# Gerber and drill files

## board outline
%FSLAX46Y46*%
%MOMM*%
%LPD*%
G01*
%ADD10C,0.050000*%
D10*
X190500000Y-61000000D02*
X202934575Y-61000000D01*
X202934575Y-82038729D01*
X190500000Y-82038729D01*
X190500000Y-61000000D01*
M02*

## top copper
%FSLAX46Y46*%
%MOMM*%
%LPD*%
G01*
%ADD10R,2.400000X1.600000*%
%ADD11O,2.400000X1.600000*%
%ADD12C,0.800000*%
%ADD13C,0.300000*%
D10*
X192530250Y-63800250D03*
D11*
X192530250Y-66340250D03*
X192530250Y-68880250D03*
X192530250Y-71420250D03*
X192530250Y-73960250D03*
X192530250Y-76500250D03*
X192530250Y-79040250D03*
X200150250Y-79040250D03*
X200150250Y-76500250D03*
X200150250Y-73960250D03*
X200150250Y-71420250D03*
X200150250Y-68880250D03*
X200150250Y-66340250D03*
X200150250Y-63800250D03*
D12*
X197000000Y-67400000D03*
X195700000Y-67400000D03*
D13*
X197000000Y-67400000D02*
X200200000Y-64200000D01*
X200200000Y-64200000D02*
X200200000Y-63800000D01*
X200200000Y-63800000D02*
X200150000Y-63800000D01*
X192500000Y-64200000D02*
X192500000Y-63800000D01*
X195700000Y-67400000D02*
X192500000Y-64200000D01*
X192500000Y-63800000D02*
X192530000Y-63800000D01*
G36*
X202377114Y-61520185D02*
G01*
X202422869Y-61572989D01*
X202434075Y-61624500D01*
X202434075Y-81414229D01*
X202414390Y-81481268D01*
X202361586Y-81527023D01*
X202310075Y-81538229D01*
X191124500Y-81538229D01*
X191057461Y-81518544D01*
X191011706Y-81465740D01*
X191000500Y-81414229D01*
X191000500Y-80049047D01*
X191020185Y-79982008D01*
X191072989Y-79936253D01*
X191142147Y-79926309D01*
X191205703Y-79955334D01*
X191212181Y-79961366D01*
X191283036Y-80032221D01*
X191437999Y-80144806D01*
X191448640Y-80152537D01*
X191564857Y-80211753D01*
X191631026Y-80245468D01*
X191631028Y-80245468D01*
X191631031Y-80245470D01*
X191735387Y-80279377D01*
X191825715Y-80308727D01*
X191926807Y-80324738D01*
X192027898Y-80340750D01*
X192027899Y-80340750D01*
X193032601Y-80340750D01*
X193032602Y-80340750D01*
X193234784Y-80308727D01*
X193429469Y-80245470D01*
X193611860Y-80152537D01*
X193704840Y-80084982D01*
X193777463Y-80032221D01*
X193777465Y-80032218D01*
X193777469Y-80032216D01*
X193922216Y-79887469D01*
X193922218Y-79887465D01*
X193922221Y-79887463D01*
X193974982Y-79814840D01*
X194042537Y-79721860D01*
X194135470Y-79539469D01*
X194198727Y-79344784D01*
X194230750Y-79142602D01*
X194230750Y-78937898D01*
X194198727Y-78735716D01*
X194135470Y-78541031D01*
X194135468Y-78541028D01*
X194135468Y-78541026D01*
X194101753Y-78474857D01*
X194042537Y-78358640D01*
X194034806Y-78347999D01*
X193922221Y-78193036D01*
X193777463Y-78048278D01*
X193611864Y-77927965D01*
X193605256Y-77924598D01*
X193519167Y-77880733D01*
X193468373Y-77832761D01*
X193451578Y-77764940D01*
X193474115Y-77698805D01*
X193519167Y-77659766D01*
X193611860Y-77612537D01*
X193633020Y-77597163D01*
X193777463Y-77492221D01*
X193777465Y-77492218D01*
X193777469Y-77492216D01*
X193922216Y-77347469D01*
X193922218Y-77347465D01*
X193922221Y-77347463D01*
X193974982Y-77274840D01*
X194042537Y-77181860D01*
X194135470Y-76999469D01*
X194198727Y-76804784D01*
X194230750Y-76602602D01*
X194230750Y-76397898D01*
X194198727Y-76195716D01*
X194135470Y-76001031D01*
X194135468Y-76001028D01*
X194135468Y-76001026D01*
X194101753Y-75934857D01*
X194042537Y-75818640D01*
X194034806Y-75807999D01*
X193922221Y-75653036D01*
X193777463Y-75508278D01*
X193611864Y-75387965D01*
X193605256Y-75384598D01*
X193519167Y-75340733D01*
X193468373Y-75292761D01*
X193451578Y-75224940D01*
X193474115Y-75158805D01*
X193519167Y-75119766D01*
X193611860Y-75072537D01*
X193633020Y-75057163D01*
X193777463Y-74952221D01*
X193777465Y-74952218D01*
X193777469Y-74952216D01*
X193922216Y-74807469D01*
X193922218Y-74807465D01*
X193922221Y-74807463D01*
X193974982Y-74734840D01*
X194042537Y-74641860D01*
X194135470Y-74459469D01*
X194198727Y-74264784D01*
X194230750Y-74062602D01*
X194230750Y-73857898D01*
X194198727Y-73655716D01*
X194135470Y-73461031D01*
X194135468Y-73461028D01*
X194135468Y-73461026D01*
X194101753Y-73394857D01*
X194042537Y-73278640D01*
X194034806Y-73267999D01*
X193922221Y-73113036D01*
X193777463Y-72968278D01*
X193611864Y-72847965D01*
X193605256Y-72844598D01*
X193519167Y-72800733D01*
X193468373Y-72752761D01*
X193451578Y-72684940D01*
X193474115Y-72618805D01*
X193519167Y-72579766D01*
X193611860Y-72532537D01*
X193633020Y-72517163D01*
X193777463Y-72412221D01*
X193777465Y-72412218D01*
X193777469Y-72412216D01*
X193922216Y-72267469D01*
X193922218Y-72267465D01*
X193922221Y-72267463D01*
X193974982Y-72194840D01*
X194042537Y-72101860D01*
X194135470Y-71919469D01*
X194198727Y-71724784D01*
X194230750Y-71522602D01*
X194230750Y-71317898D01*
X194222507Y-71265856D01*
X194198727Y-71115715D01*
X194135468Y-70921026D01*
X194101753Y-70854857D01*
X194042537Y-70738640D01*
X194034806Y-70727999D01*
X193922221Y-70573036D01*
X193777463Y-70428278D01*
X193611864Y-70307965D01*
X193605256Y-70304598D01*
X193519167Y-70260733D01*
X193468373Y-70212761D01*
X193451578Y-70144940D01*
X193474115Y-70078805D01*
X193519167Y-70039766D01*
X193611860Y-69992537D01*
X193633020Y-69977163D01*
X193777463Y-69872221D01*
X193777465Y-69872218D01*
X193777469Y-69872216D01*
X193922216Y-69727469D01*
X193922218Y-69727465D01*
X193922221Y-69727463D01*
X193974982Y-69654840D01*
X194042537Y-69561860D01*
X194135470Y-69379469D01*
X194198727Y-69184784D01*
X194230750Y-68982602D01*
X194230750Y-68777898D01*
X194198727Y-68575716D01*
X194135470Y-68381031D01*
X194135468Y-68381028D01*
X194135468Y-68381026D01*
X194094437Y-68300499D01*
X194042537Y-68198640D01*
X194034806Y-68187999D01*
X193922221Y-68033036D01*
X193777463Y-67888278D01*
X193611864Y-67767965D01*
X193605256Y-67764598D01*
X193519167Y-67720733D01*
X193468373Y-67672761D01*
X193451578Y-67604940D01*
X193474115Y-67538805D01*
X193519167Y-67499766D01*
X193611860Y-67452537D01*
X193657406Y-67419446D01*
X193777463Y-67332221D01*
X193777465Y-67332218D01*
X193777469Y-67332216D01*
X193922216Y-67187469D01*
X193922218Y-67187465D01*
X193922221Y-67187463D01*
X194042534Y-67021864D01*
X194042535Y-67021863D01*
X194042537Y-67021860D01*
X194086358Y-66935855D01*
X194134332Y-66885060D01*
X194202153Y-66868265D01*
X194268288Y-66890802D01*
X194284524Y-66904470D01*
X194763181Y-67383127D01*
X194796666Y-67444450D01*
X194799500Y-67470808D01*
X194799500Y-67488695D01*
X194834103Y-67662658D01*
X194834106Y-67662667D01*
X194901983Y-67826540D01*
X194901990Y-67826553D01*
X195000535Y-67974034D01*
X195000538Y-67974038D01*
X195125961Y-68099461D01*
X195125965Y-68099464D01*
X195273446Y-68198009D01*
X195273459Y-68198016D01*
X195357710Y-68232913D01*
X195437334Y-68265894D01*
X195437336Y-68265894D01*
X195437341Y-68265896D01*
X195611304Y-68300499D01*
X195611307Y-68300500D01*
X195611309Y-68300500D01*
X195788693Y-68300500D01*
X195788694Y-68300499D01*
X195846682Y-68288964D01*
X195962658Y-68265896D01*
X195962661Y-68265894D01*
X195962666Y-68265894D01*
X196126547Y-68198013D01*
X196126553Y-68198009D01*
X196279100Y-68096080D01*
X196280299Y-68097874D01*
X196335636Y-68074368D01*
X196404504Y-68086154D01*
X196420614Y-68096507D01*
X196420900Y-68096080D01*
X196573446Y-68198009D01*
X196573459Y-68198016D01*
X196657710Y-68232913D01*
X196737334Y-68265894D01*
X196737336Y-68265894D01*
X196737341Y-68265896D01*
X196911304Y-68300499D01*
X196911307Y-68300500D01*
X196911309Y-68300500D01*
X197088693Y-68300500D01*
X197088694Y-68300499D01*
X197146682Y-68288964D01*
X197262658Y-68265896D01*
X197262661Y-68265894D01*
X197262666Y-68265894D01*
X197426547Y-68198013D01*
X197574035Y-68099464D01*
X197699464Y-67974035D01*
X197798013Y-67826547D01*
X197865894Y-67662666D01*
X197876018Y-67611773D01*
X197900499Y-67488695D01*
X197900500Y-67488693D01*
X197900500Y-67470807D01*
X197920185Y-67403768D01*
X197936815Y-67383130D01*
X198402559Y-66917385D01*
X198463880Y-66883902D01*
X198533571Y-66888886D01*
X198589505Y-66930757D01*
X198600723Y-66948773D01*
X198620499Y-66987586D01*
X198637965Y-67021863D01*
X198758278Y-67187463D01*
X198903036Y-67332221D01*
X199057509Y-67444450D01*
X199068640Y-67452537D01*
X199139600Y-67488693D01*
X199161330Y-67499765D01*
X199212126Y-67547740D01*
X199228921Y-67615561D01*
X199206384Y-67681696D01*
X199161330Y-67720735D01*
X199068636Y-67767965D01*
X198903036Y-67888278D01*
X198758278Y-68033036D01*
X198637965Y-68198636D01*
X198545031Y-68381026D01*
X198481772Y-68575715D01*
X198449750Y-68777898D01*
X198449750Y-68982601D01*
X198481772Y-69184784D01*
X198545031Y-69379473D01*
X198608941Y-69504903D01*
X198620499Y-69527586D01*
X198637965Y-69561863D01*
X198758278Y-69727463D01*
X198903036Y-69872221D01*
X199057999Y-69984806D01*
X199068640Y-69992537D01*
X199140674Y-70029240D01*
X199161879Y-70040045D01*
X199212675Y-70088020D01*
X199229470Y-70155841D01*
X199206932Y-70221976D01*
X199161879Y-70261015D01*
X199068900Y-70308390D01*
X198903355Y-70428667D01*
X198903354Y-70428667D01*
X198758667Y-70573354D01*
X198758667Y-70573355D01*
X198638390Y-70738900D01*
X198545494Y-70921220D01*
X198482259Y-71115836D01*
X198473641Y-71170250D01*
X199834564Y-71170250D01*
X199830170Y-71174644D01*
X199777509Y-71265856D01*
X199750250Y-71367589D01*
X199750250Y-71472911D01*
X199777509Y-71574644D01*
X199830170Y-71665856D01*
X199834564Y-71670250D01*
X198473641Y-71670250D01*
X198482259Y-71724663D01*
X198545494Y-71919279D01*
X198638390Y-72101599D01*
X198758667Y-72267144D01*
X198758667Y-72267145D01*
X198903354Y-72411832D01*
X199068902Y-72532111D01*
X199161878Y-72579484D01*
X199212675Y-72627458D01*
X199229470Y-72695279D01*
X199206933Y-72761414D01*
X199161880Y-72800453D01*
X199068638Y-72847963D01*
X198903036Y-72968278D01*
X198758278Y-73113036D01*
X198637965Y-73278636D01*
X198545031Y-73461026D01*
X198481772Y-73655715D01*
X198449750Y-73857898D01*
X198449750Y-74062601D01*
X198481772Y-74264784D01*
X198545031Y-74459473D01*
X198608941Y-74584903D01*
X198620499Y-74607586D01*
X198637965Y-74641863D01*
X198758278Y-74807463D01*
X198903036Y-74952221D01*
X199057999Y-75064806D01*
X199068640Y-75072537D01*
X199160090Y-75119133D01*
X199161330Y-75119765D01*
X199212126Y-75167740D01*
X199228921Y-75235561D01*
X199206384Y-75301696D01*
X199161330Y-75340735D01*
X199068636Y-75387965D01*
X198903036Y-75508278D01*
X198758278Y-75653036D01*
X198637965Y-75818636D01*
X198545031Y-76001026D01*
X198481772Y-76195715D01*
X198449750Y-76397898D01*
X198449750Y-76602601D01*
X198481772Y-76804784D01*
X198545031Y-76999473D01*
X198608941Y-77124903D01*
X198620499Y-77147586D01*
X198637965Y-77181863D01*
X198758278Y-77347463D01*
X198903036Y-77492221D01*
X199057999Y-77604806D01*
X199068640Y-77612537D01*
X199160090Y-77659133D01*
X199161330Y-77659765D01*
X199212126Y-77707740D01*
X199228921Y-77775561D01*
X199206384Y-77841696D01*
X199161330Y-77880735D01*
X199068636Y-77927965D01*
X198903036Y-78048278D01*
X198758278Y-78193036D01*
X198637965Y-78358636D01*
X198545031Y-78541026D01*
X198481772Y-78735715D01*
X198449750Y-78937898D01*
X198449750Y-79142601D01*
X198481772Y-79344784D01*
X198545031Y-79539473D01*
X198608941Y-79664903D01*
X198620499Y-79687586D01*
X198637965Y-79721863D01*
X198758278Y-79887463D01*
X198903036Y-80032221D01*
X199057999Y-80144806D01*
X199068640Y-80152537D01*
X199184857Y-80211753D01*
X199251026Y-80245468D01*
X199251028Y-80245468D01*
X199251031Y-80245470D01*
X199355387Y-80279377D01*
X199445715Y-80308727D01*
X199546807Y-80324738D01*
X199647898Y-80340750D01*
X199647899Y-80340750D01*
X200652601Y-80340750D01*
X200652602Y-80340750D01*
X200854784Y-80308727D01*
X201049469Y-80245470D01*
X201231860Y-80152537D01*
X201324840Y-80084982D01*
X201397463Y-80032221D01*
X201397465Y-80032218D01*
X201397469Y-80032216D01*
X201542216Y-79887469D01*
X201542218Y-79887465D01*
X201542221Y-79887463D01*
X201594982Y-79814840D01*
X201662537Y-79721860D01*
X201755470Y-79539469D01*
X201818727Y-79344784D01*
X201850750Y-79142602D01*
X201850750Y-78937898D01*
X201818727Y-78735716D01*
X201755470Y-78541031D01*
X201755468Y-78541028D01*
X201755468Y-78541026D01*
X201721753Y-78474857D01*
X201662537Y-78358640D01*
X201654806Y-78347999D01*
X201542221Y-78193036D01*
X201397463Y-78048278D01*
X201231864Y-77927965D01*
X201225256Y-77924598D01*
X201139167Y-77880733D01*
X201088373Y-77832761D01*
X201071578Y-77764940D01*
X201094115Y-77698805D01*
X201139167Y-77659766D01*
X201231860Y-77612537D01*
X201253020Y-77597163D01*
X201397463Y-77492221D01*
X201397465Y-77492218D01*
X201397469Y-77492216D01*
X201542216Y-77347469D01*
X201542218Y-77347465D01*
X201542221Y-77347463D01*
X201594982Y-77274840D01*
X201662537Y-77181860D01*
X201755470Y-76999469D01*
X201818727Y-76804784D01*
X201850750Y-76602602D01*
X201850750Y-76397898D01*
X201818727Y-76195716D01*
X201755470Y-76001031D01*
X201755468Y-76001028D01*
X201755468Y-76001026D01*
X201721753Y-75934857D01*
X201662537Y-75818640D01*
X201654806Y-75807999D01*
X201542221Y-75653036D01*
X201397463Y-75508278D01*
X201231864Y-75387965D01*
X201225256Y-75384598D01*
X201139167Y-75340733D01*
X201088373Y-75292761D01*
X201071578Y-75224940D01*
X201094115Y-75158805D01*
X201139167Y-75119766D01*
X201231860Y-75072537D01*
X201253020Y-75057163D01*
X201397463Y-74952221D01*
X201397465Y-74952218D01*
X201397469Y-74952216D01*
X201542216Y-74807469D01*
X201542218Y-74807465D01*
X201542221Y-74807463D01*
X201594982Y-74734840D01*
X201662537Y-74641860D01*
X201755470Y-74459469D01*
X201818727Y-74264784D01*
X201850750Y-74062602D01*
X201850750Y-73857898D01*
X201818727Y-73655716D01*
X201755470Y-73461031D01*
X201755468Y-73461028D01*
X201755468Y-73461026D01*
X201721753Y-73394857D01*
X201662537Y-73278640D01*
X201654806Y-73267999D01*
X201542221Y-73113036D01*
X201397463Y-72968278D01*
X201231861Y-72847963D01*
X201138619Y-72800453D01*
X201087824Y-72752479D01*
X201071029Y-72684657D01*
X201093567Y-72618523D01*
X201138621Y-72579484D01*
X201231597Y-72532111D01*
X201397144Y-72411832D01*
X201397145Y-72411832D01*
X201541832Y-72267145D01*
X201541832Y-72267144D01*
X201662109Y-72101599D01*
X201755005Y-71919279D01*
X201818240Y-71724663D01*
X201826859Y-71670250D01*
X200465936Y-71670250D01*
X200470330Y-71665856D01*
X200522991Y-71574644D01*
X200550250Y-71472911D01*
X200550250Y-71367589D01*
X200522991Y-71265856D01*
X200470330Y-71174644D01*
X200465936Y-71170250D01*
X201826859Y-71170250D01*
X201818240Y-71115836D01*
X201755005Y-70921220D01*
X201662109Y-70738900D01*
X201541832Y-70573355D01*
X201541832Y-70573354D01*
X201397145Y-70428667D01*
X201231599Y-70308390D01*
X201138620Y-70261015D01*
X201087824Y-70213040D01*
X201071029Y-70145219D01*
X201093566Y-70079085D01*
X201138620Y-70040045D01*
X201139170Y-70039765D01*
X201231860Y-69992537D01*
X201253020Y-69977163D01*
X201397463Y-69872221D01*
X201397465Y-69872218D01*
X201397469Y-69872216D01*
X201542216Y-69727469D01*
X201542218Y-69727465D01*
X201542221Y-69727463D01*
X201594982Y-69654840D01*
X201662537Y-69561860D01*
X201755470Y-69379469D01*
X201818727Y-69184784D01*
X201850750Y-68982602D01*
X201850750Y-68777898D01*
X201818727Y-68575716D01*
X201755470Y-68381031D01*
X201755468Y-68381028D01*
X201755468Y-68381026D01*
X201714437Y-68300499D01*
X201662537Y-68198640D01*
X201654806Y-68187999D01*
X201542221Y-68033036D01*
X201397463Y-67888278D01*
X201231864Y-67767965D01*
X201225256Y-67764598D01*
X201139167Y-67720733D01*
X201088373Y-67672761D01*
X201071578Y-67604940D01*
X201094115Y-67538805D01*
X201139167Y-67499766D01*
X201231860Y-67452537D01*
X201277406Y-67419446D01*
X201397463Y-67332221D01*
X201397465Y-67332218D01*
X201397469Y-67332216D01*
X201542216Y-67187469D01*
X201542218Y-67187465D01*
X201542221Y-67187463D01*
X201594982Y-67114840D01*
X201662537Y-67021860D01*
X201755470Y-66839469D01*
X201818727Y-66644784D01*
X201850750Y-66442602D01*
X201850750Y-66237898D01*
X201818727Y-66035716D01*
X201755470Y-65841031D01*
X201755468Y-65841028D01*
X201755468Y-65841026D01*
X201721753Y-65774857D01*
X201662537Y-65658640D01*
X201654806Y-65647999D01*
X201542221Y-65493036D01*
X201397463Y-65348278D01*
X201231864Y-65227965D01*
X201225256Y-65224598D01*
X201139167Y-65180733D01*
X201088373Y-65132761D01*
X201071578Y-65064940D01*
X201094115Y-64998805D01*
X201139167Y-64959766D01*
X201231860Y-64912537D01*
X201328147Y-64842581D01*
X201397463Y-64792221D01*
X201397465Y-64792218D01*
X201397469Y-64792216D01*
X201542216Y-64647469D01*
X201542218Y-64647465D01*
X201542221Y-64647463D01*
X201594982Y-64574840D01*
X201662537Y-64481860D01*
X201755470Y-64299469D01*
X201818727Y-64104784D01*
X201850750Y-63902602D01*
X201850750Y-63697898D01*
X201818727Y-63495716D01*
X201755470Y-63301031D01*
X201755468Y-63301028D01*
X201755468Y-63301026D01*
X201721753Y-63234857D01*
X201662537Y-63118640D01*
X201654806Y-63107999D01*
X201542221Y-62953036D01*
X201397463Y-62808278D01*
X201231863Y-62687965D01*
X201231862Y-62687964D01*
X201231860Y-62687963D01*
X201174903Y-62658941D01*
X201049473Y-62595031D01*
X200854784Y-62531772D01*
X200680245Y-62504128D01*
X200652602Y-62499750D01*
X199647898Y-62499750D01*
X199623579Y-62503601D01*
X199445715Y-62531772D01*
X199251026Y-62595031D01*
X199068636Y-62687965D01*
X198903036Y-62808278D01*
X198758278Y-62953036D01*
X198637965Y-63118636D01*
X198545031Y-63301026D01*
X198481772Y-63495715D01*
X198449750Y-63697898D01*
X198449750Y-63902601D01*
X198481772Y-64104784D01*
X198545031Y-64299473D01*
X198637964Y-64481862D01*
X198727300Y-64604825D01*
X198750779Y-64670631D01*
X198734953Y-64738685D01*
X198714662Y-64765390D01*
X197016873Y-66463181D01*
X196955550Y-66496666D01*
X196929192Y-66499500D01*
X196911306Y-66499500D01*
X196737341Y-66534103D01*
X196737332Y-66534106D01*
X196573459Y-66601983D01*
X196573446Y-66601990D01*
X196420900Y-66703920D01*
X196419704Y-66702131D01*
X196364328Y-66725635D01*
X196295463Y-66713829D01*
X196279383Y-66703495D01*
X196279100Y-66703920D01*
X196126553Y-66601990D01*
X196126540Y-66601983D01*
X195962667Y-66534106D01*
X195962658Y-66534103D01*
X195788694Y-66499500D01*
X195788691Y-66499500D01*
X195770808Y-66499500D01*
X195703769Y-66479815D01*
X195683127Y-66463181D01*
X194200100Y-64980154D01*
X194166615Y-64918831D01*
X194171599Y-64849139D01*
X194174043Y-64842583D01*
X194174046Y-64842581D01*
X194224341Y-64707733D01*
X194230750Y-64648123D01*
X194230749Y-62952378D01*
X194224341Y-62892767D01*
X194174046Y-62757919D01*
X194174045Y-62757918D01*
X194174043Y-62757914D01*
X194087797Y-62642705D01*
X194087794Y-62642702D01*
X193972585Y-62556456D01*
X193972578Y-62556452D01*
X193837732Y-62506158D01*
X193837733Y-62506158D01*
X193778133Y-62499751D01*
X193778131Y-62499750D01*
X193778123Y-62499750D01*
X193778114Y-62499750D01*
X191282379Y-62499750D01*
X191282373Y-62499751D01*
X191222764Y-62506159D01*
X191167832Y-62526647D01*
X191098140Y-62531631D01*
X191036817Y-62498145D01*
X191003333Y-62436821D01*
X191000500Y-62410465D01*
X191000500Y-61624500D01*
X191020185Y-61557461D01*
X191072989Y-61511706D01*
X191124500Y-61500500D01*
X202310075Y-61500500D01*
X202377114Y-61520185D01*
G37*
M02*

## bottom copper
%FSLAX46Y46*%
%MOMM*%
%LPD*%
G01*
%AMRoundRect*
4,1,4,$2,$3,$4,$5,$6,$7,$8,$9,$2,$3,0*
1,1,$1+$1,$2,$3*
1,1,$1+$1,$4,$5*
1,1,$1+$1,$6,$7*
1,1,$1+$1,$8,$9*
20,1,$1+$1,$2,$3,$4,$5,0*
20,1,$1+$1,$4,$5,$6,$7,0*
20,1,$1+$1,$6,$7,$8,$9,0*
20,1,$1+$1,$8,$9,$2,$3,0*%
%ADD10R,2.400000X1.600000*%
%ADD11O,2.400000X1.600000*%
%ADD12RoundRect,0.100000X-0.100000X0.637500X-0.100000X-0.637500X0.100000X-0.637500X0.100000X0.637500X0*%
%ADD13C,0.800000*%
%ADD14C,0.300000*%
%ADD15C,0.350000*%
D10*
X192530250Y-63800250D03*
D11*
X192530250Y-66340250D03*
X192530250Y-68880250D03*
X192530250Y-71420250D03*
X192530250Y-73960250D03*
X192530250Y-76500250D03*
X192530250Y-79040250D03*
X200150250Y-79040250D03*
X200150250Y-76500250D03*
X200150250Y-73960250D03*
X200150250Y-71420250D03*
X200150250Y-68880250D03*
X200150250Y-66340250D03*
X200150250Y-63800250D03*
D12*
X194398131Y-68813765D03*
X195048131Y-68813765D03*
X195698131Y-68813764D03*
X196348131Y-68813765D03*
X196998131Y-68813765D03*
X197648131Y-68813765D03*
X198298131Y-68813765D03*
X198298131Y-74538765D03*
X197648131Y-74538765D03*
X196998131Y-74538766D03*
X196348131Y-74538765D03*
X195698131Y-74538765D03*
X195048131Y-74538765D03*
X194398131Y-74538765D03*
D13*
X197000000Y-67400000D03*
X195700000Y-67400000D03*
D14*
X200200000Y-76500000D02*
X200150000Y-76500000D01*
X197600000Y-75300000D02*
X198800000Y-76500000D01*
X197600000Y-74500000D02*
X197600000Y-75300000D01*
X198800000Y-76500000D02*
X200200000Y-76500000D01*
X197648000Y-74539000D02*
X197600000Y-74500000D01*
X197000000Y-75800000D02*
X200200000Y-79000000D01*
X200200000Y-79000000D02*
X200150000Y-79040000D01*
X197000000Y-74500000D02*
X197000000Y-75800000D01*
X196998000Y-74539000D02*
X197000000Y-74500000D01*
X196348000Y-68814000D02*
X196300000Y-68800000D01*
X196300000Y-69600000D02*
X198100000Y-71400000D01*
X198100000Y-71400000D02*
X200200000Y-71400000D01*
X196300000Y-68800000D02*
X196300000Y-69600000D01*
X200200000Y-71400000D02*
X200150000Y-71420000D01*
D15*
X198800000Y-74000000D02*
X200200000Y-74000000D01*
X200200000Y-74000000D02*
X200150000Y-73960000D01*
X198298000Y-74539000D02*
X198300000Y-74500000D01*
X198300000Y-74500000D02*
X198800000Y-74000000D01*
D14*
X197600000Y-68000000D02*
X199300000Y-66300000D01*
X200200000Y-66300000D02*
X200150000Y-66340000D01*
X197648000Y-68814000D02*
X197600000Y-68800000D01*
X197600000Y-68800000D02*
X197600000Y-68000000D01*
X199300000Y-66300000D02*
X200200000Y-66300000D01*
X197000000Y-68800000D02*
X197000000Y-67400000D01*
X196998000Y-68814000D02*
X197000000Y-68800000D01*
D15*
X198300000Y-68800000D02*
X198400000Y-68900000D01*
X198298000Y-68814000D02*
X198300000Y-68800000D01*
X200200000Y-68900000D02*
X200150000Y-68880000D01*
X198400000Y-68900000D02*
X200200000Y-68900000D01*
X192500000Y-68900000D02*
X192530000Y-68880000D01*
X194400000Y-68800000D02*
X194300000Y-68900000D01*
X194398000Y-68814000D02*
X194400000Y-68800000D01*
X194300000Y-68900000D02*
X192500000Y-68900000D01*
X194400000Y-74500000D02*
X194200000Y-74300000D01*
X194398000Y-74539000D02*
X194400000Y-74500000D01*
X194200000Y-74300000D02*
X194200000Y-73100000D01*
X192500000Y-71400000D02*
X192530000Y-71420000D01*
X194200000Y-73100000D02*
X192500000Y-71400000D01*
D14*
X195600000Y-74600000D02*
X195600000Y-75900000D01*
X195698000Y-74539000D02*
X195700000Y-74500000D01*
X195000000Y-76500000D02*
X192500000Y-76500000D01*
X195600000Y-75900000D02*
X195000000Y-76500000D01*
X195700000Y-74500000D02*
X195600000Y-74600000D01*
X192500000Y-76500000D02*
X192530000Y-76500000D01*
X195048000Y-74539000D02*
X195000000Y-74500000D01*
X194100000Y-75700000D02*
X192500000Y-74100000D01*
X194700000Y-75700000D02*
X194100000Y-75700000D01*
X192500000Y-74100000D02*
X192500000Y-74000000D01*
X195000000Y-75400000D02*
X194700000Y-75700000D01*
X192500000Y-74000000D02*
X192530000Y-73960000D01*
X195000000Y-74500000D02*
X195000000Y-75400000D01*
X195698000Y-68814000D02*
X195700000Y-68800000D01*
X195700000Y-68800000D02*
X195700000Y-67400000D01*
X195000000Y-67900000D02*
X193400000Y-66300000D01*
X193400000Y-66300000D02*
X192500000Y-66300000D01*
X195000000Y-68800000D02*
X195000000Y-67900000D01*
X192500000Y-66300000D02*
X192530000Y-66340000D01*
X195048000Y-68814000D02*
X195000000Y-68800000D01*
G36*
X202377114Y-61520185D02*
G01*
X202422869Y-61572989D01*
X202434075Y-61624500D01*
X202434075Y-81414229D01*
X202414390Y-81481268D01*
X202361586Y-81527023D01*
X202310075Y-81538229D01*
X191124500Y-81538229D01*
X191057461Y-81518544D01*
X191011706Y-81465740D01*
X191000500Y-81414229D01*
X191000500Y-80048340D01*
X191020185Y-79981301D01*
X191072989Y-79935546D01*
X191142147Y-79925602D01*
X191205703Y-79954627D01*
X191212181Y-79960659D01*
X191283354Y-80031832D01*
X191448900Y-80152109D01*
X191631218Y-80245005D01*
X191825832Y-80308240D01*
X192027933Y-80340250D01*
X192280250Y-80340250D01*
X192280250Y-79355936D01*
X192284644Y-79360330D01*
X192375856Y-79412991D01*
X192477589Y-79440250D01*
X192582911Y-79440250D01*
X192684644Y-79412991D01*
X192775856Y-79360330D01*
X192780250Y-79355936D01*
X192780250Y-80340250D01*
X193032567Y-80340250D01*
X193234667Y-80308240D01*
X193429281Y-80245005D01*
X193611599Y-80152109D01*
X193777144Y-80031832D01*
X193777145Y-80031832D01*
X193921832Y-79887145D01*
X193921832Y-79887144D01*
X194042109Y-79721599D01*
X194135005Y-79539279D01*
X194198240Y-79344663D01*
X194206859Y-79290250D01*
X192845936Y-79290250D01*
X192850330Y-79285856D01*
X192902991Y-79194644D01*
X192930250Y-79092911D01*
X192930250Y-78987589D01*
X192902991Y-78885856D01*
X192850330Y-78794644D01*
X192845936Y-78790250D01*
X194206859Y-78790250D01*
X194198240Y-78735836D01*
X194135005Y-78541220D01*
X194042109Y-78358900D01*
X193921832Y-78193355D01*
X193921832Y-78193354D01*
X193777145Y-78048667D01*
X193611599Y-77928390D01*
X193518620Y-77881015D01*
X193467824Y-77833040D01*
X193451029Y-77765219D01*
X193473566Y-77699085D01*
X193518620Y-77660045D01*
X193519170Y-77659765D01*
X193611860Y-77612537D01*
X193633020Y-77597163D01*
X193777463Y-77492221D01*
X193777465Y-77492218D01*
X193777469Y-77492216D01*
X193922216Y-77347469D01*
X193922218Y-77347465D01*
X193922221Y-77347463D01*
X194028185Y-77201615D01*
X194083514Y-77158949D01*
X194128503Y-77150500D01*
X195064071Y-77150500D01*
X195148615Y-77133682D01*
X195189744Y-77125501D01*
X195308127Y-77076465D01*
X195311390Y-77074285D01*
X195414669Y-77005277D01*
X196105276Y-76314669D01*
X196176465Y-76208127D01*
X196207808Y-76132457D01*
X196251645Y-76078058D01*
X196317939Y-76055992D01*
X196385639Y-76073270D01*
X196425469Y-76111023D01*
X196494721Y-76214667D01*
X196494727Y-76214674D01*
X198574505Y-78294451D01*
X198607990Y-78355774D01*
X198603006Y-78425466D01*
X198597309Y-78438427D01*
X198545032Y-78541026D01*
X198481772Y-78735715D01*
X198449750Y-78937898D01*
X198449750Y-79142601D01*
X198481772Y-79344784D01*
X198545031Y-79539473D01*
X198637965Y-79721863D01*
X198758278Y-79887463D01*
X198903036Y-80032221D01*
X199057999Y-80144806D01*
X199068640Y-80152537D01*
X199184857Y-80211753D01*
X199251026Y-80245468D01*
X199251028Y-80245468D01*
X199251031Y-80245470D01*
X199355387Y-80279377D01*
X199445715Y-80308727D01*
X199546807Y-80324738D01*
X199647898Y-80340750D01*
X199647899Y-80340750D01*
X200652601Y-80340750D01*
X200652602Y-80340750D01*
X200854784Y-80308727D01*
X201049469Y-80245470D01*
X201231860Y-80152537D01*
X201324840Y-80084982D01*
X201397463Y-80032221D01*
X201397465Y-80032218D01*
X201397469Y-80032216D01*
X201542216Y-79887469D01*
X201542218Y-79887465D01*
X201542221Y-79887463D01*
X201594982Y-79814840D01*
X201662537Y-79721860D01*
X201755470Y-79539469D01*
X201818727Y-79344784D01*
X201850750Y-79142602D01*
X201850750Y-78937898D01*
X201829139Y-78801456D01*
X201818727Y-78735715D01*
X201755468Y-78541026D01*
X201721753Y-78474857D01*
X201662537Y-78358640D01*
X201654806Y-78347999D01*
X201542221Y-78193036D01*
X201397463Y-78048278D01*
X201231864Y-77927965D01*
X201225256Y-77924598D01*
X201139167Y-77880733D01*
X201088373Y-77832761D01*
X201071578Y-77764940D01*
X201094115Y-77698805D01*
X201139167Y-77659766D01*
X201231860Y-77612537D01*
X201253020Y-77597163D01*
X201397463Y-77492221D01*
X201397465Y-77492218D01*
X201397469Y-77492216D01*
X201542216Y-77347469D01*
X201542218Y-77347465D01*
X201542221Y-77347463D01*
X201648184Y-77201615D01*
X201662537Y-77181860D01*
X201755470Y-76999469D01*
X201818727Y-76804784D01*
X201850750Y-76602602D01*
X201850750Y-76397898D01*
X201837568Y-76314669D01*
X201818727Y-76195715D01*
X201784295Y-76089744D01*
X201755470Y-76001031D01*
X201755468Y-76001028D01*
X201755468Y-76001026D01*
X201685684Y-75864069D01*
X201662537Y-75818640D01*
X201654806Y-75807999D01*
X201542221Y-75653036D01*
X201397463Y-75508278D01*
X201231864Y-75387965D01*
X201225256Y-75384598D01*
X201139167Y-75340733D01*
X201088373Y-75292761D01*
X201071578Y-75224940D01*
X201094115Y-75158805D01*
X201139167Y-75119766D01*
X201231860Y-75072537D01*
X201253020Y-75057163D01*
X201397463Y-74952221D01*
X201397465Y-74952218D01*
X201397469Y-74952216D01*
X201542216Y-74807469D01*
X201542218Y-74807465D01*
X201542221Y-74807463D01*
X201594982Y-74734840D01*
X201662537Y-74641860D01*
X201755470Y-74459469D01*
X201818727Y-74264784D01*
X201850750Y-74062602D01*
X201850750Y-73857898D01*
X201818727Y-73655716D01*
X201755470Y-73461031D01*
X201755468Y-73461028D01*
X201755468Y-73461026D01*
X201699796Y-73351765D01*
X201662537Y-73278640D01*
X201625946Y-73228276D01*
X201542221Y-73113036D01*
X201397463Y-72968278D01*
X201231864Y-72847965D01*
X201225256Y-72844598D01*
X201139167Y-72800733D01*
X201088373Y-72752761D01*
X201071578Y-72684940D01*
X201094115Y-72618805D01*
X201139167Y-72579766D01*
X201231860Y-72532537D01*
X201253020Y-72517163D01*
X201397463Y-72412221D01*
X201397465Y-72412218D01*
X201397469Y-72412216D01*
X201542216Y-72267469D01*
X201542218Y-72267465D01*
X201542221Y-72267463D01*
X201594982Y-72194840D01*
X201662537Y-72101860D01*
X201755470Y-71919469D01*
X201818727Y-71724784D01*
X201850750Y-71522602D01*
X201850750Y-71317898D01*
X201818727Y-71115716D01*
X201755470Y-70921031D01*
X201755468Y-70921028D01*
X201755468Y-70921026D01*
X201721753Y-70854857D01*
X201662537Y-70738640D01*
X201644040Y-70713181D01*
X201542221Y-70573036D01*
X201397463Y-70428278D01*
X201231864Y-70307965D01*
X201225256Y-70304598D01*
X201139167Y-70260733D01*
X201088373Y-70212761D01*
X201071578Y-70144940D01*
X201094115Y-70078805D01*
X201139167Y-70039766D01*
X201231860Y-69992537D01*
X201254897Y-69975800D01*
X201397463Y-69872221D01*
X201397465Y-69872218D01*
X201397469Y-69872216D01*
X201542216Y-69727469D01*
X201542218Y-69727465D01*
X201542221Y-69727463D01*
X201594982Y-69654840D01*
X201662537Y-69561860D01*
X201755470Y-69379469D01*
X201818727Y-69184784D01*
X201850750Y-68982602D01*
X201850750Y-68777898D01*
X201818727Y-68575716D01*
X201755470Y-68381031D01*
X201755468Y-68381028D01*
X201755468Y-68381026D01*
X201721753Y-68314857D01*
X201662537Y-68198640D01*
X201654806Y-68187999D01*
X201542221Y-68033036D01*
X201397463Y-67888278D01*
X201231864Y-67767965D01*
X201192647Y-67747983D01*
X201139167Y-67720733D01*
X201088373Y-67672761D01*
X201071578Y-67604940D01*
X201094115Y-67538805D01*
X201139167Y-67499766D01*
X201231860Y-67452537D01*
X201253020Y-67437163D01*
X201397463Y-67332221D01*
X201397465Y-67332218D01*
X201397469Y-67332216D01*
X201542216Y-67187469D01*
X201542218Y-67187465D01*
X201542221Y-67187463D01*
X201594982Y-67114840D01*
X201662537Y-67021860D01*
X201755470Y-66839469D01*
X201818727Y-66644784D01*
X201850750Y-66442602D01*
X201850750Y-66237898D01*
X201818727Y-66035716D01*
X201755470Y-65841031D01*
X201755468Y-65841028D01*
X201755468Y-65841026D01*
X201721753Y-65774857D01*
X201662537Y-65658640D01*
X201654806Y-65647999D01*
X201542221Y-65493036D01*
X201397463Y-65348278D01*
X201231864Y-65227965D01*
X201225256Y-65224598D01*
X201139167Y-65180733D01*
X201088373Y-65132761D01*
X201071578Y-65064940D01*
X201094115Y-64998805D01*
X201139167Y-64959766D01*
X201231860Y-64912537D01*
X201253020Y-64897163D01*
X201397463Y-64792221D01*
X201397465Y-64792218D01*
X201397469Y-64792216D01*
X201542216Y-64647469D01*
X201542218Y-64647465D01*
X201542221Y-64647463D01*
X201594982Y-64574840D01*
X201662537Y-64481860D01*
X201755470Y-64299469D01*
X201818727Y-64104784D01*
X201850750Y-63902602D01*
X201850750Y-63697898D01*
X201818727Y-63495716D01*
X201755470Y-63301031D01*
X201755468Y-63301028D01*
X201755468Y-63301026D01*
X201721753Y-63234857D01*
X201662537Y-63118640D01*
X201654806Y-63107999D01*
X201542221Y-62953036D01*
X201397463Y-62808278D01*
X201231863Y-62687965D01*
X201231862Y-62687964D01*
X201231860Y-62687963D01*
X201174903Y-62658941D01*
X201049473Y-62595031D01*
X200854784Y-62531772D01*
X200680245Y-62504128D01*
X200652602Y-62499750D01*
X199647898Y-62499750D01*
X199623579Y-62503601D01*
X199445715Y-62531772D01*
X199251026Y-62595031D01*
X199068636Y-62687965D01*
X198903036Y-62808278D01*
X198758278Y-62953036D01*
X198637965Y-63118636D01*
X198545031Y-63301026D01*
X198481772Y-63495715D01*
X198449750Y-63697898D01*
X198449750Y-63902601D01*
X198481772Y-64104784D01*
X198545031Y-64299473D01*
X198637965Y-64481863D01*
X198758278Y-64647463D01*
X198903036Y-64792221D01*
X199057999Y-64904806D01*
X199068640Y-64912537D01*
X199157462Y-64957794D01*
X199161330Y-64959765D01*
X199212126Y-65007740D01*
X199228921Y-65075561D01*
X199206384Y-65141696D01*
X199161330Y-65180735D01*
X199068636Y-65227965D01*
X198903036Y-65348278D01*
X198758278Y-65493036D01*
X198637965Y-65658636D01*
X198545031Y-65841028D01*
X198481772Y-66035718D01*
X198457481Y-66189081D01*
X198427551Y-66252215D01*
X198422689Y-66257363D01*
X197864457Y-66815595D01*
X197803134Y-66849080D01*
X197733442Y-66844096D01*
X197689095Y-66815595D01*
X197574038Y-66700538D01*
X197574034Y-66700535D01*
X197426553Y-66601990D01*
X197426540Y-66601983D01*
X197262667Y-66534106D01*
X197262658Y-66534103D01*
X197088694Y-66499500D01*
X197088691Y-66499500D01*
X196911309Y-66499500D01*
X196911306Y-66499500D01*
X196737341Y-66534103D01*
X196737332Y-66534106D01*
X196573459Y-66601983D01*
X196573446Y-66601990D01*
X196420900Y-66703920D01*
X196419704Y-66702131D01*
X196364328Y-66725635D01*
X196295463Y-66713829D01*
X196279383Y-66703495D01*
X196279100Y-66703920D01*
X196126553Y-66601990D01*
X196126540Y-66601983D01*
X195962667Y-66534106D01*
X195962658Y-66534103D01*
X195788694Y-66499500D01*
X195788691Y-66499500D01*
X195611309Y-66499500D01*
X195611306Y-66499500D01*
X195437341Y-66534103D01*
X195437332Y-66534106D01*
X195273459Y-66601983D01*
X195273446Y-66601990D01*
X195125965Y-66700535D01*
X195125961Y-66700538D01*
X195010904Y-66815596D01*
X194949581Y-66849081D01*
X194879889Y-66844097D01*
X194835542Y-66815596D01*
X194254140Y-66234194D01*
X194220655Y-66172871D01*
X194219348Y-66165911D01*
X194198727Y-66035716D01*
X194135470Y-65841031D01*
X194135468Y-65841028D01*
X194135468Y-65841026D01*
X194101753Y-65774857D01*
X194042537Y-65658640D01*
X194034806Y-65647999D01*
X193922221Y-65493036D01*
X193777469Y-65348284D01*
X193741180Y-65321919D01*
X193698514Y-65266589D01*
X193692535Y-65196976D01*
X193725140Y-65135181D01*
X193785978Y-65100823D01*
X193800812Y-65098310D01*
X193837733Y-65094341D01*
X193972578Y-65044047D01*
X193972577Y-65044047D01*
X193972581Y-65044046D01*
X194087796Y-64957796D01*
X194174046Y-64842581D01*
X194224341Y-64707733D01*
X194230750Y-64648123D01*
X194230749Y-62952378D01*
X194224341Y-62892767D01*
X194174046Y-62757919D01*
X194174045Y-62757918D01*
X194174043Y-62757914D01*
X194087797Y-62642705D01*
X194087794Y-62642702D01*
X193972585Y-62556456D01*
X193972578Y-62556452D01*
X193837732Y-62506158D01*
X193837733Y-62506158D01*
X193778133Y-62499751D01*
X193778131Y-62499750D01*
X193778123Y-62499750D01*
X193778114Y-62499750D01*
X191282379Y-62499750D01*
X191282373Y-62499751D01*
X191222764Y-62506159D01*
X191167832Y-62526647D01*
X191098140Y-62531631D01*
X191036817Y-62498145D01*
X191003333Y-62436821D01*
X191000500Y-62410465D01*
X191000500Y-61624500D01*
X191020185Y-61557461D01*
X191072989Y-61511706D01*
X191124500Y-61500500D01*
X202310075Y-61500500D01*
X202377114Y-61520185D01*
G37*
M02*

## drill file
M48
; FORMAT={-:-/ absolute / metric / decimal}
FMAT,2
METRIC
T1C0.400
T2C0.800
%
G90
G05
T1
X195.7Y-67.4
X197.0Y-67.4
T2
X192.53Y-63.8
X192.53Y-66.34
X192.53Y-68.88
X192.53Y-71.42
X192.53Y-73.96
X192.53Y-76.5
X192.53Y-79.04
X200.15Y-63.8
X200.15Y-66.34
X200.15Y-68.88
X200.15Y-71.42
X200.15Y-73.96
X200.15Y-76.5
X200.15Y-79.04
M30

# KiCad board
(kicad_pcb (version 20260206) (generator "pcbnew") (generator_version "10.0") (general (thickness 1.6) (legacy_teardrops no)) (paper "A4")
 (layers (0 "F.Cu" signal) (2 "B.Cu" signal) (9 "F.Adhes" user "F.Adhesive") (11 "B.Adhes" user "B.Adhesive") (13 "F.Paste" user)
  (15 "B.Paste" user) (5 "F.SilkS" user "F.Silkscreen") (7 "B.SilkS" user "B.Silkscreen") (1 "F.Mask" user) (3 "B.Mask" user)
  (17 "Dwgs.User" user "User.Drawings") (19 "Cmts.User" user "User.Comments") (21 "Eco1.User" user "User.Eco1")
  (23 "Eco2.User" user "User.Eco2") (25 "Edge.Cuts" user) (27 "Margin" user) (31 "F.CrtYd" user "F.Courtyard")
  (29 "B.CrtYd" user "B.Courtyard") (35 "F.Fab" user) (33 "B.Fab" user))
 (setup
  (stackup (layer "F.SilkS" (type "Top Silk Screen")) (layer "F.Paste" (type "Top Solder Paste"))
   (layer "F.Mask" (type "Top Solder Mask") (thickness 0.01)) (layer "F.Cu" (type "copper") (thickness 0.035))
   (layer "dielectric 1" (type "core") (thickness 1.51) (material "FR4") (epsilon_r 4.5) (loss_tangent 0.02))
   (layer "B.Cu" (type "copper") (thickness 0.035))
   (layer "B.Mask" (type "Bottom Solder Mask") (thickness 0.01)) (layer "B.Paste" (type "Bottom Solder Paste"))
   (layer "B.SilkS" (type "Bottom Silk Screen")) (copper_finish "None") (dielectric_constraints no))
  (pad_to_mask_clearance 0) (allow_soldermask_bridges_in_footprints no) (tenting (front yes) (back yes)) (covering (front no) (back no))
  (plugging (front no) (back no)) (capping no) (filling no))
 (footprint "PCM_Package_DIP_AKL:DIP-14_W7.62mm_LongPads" (layer "F.Cu") (at 192.53025 63.80025)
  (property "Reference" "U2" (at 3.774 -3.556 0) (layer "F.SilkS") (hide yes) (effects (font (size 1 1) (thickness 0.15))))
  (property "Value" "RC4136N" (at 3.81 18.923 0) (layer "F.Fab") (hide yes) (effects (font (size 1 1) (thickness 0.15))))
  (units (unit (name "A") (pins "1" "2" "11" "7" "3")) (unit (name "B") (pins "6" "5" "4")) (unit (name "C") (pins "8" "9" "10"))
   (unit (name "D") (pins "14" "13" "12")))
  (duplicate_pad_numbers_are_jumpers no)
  (pad "1" thru_hole rect (at 0 0) (size 2.4 1.6) (drill 0.8) (layers "*.Cu" "*.Mask") (remove_unused_layers no) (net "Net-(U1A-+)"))
  (pad "2" thru_hole oval (at 0 2.54) (size 2.4 1.6) (drill 0.8) (layers "*.Cu" "*.Mask") (remove_unused_layers no) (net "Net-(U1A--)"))
  (pad "3" thru_hole oval (at 0 5.08) (size 2.4 1.6) (drill 0.8) (layers "*.Cu" "*.Mask") (remove_unused_layers no) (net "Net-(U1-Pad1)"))
  (pad "4" thru_hole oval (at 0 7.62) (size 2.4 1.6) (drill 0.8) (layers "*.Cu" "*.Mask") (remove_unused_layers no) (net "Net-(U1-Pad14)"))
  (pad "5" thru_hole oval (at 0 10.16) (size 2.4 1.6) (drill 0.8) (layers "*.Cu" "*.Mask") (remove_unused_layers no) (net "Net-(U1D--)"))
  (pad "6" thru_hole oval (at 0 12.7) (size 2.4 1.6) (drill 0.8) (layers "*.Cu" "*.Mask") (remove_unused_layers no) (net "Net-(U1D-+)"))
  (pad "7" thru_hole oval (at 0 15.24) (size 2.4 1.6) (drill 0.8) (layers "*.Cu" "*.Mask") (remove_unused_layers no) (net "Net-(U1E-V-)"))
  (pad "8" thru_hole oval (at 7.62 15.24) (size 2.4 1.6) (drill 0.8) (layers "*.Cu" "*.Mask") (remove_unused_layers no) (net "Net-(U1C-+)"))
  (pad "9" thru_hole oval (at 7.62 12.7) (size 2.4 1.6) (drill 0.8) (layers "*.Cu" "*.Mask") (remove_unused_layers no) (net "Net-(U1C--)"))
  (pad "10" thru_hole oval (at 7.62 10.16) (size 2.4 1.6) (drill 0.8) (layers "*.Cu" "*.Mask") (remove_unused_layers no)
   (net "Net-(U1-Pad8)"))
  (pad "11" thru_hole oval (at 7.62 7.62) (size 2.4 1.6) (drill 0.8) (layers "*.Cu" "*.Mask") (remove_unused_layers no) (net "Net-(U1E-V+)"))
  (pad "12" thru_hole oval (at 7.62 5.08) (size 2.4 1.6) (drill 0.8) (layers "*.Cu" "*.Mask") (remove_unused_layers no)
   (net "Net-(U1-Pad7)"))
  (pad "13" thru_hole oval (at 7.62 2.54) (size 2.4 1.6) (drill 0.8) (layers "*.Cu" "*.Mask") (remove_unused_layers no) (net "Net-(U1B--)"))
  (pad "14" thru_hole oval (at 7.62 0) (size 2.4 1.6) (drill 0.8) (layers "*.Cu" "*.Mask") (remove_unused_layers no) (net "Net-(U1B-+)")))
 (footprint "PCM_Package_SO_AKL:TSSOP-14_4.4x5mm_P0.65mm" (layer "B.Cu") (at 196.348131 71.676265 -90)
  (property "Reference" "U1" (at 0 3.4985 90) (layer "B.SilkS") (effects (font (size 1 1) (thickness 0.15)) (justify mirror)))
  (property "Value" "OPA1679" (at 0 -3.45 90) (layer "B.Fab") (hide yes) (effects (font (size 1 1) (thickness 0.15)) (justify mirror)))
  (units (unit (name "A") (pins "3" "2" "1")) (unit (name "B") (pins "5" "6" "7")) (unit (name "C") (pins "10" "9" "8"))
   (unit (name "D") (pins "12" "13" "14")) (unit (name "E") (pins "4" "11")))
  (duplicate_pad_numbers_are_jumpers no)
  (pad "1" smd roundrect (at -2.8625 1.95 270) (size 1.475 0.4) (layers "B.Cu" "B.Mask" "B.Paste") (roundrect_rratio 0.25)
   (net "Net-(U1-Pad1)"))
  (pad "2" smd roundrect (at -2.8625 1.3 270) (size 1.475 0.4) (layers "B.Cu" "B.Mask" "B.Paste") (roundrect_rratio 0.25)
   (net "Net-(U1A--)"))
  (pad "3" smd roundrect (at -2.862501 0.65 270) (size 1.475 0.4) (layers "B.Cu" "B.Mask" "B.Paste") (roundrect_rratio 0.25)
   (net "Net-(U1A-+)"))
  (pad "4" smd roundrect (at -2.8625 0 270) (size 1.475 0.4) (layers "B.Cu" "B.Mask" "B.Paste") (roundrect_rratio 0.25) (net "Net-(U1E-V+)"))
  (pad "5" smd roundrect (at -2.8625 -0.65 270) (size 1.475 0.4) (layers "B.Cu" "B.Mask" "B.Paste") (roundrect_rratio 0.25)
   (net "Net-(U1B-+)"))
  (pad "6" smd roundrect (at -2.8625 -1.3 270) (size 1.475 0.4) (layers "B.Cu" "B.Mask" "B.Paste") (roundrect_rratio 0.25)
   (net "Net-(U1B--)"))
  (pad "7" smd roundrect (at -2.8625 -1.95 270) (size 1.475 0.4) (layers "B.Cu" "B.Mask" "B.Paste") (roundrect_rratio 0.25)
   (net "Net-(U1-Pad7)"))
  (pad "8" smd roundrect (at 2.8625 -1.95 270) (size 1.475 0.4) (layers "B.Cu" "B.Mask" "B.Paste") (roundrect_rratio 0.25)
   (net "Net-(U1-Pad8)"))
  (pad "9" smd roundrect (at 2.8625 -1.3 270) (size 1.475 0.4) (layers "B.Cu" "B.Mask" "B.Paste") (roundrect_rratio 0.25)
   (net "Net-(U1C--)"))
  (pad "10" smd roundrect (at 2.862501 -0.65 270) (size 1.475 0.4) (layers "B.Cu" "B.Mask" "B.Paste") (roundrect_rratio 0.25)
   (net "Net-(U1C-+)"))
  (pad "11" smd roundrect (at 2.8625 0 270) (size 1.475 0.4) (layers "B.Cu" "B.Mask" "B.Paste") (roundrect_rratio 0.25) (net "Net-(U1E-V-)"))
  (pad "12" smd roundrect (at 2.8625 0.65 270) (size 1.475 0.4) (layers "B.Cu" "B.Mask" "B.Paste") (roundrect_rratio 0.25)
   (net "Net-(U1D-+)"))
  (pad "13" smd roundrect (at 2.8625 1.3 270) (size 1.475 0.4) (layers "B.Cu" "B.Mask" "B.Paste") (roundrect_rratio 0.25)
   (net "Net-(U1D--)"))
  (pad "14" smd roundrect (at 2.8625 1.95 270) (size 1.475 0.4) (layers "B.Cu" "B.Mask" "B.Paste") (roundrect_rratio 0.25)
   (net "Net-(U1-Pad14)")))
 (gr_rect (start 190.5 61) (end 202.934575 82.038729) (stroke (width 0.05) (type default)) (fill no) (layer "Edge.Cuts"))
 (segment (start 200.2 76.5) (end 200.15 76.5) (width 0.3) (layer "B.Cu") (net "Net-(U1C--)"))
 (segment (start 197.6 75.3) (end 198.8 76.5) (width 0.3) (layer "B.Cu") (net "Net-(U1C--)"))
 (segment (start 197.6 74.5) (end 197.6 75.3) (width 0.3) (layer "B.Cu") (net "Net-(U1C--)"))
 (segment (start 198.8 76.5) (end 200.2 76.5) (width 0.3) (layer "B.Cu") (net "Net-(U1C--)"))
 (segment (start 197.648 74.539) (end 197.6 74.5) (width 0.3) (layer "B.Cu") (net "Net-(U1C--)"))
 (segment (start 197 75.8) (end 200.2 79) (width 0.3) (layer "B.Cu") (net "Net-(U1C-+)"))
 (segment (start 200.2 79) (end 200.15 79.04) (width 0.3) (layer "B.Cu") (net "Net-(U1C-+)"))
 (segment (start 197 74.5) (end 197 75.8) (width 0.3) (layer "B.Cu") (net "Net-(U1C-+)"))
 (segment (start 196.998 74.539) (end 197 74.5) (width 0.3) (layer "B.Cu") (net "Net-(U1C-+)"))
 (segment (start 196.348 68.814) (end 196.3 68.8) (width 0.3) (layer "B.Cu") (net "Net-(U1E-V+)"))
 (segment (start 196.3 69.6) (end 198.1 71.4) (width 0.3) (layer "B.Cu") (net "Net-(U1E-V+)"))
 (segment (start 198.1 71.4) (end 200.2 71.4) (width 0.3) (layer "B.Cu") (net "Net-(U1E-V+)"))
 (segment (start 196.3 68.8) (end 196.3 69.6) (width 0.3) (layer "B.Cu") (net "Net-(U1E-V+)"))
 (segment (start 200.2 71.4) (end 200.15 71.42) (width 0.3) (layer "B.Cu") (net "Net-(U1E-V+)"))
 (segment (start 198.8 74) (end 200.2 74) (width 0.35) (layer "B.Cu") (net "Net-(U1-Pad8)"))
 (segment (start 200.2 74) (end 200.15 73.96) (width 0.35) (layer "B.Cu") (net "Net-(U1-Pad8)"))
 (segment (start 198.298 74.539) (end 198.3 74.5) (width 0.35) (layer "B.Cu") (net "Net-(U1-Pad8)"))
 (segment (start 198.3 74.5) (end 198.8 74) (width 0.35) (layer "B.Cu") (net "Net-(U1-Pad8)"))
 (segment (start 197.6 68) (end 199.3 66.3) (width 0.3) (layer "B.Cu") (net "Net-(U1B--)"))
 (segment (start 200.2 66.3) (end 200.15 66.34) (width 0.3) (layer "B.Cu") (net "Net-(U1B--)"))
 (segment (start 197.648 68.814) (end 197.6 68.8) (width 0.3) (layer "B.Cu") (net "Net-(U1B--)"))
 (segment (start 197.6 68.8) (end 197.6 68) (width 0.3) (layer "B.Cu") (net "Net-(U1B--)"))
 (segment (start 199.3 66.3) (end 200.2 66.3) (width 0.3) (layer "B.Cu") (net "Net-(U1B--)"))
 (segment (start 197 67.4) (end 200.2 64.2) (width 0.3) (layer "F.Cu") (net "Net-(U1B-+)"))
 (segment (start 200.2 64.2) (end 200.2 63.8) (width 0.3) (layer "F.Cu") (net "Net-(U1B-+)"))
 (segment (start 200.2 63.8) (end 200.15 63.8) (width 0.3) (layer "F.Cu") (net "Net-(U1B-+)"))
 (via (at 197 67.4) (size 0.8) (drill 0.4) (layers "F.Cu" "B.Cu") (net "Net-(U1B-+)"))
 (segment (start 197 68.8) (end 197 67.4) (width 0.3) (layer "B.Cu") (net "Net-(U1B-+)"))
 (segment (start 196.998 68.814) (end 197 68.8) (width 0.3) (layer "B.Cu") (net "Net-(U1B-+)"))
 (segment (start 198.3 68.8) (end 198.4 68.9) (width 0.35) (layer "B.Cu") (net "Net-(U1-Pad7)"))
 (segment (start 198.298 68.814) (end 198.3 68.8) (width 0.35) (layer "B.Cu") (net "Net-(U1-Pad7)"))
 (segment (start 200.2 68.9) (end 200.15 68.88) (width 0.35) (layer "B.Cu") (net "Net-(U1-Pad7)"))
 (segment (start 198.4 68.9) (end 200.2 68.9) (width 0.35) (layer "B.Cu") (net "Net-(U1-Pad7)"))
 (segment (start 192.5 68.9) (end 192.53 68.88) (width 0.35) (layer "B.Cu") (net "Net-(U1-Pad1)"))
 (segment (start 194.4 68.8) (end 194.3 68.9) (width 0.35) (layer "B.Cu") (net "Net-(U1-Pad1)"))
 (segment (start 194.398 68.814) (end 194.4 68.8) (width 0.35) (layer "B.Cu") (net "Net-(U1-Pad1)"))
 (segment (start 194.3 68.9) (end 192.5 68.9) (width 0.35) (layer "B.Cu") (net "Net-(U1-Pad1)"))
 (segment (start 194.4 74.5) (end 194.2 74.3) (width 0.35) (layer "B.Cu") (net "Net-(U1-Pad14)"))
 (segment (start 194.398 74.539) (end 194.4 74.5) (width 0.35) (layer "B.Cu") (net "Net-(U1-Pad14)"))
 (segment (start 194.2 74.3) (end 194.2 73.1) (width 0.35) (layer "B.Cu") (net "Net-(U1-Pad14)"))
 (segment (start 192.5 71.4) (end 192.53 71.42) (width 0.35) (layer "B.Cu") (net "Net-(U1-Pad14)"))
 (segment (start 194.2 73.1) (end 192.5 71.4) (width 0.35) (layer "B.Cu") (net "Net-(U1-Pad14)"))
 (segment (start 195.6 74.6) (end 195.6 75.9) (width 0.3) (layer "B.Cu") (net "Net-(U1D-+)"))
 (segment (start 195.698 74.539) (end 195.7 74.5) (width 0.3) (layer "B.Cu") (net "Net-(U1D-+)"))
 (segment (start 195 76.5) (end 192.5 76.5) (width 0.3) (layer "B.Cu") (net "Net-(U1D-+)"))
 (segment (start 195.6 75.9) (end 195 76.5) (width 0.3) (layer "B.Cu") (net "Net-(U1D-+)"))
 (segment (start 195.7 74.5) (end 195.6 74.6) (width 0.3) (layer "B.Cu") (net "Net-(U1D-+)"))
 (segment (start 192.5 76.5) (end 192.53 76.5) (width 0.3) (layer "B.Cu") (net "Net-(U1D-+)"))
 (segment (start 195.048 74.539) (end 195 74.5) (width 0.3) (layer "B.Cu") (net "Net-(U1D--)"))
 (segment (start 194.1 75.7) (end 192.5 74.1) (width 0.3) (layer "B.Cu") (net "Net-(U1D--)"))
 (segment (start 194.7 75.7) (end 194.1 75.7) (width 0.3) (layer "B.Cu") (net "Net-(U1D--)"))
 (segment (start 192.5 74.1) (end 192.5 74) (width 0.3) (layer "B.Cu") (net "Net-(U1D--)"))
 (segment (start 195 75.4) (end 194.7 75.7) (width 0.3) (layer "B.Cu") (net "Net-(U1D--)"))
 (segment (start 192.5 74) (end 192.53 73.96) (width 0.3) (layer "B.Cu") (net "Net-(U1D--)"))
 (segment (start 195 74.5) (end 195 75.4) (width 0.3) (layer "B.Cu") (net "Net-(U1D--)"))
 (segment (start 192.5 64.2) (end 192.5 63.8) (width 0.3) (layer "F.Cu") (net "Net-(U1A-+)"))
 (segment (start 195.7 67.4) (end 192.5 64.2) (width 0.3) (layer "F.Cu") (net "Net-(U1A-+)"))
 (segment (start 192.5 63.8) (end 192.53 63.8) (width 0.3) (layer "F.Cu") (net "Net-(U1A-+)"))
 (via (at 195.7 67.4) (size 0.8) (drill 0.4) (layers "F.Cu" "B.Cu") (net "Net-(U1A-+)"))
 (segment (start 195.698 68.814) (end 195.7 68.8) (width 0.3) (layer "B.Cu") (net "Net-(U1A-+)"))
 (segment (start 195.7 68.8) (end 195.7 67.4) (width 0.3) (layer "B.Cu") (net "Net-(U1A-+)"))
 (segment (start 195 67.9) (end 193.4 66.3) (width 0.3) (layer "B.Cu") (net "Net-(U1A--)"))
 (segment (start 193.4 66.3) (end 192.5 66.3) (width 0.3) (layer "B.Cu") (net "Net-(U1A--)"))
 (segment (start 195 68.8) (end 195 67.9) (width 0.3) (layer "B.Cu") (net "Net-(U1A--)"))
 (segment (start 192.5 66.3) (end 192.53 66.34) (width 0.3) (layer "B.Cu") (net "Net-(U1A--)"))
 (segment (start 195.048 68.814) (end 195 68.8) (width 0.3) (layer "B.Cu") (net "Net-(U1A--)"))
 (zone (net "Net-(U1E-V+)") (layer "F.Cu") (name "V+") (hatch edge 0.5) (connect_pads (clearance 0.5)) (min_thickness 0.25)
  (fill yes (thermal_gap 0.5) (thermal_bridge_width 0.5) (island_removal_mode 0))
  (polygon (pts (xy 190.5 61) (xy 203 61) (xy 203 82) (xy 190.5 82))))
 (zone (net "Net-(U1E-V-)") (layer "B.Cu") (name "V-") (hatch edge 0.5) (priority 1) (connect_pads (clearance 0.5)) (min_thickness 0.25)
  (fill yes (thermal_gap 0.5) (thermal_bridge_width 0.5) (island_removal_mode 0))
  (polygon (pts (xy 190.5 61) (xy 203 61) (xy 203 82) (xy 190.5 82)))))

